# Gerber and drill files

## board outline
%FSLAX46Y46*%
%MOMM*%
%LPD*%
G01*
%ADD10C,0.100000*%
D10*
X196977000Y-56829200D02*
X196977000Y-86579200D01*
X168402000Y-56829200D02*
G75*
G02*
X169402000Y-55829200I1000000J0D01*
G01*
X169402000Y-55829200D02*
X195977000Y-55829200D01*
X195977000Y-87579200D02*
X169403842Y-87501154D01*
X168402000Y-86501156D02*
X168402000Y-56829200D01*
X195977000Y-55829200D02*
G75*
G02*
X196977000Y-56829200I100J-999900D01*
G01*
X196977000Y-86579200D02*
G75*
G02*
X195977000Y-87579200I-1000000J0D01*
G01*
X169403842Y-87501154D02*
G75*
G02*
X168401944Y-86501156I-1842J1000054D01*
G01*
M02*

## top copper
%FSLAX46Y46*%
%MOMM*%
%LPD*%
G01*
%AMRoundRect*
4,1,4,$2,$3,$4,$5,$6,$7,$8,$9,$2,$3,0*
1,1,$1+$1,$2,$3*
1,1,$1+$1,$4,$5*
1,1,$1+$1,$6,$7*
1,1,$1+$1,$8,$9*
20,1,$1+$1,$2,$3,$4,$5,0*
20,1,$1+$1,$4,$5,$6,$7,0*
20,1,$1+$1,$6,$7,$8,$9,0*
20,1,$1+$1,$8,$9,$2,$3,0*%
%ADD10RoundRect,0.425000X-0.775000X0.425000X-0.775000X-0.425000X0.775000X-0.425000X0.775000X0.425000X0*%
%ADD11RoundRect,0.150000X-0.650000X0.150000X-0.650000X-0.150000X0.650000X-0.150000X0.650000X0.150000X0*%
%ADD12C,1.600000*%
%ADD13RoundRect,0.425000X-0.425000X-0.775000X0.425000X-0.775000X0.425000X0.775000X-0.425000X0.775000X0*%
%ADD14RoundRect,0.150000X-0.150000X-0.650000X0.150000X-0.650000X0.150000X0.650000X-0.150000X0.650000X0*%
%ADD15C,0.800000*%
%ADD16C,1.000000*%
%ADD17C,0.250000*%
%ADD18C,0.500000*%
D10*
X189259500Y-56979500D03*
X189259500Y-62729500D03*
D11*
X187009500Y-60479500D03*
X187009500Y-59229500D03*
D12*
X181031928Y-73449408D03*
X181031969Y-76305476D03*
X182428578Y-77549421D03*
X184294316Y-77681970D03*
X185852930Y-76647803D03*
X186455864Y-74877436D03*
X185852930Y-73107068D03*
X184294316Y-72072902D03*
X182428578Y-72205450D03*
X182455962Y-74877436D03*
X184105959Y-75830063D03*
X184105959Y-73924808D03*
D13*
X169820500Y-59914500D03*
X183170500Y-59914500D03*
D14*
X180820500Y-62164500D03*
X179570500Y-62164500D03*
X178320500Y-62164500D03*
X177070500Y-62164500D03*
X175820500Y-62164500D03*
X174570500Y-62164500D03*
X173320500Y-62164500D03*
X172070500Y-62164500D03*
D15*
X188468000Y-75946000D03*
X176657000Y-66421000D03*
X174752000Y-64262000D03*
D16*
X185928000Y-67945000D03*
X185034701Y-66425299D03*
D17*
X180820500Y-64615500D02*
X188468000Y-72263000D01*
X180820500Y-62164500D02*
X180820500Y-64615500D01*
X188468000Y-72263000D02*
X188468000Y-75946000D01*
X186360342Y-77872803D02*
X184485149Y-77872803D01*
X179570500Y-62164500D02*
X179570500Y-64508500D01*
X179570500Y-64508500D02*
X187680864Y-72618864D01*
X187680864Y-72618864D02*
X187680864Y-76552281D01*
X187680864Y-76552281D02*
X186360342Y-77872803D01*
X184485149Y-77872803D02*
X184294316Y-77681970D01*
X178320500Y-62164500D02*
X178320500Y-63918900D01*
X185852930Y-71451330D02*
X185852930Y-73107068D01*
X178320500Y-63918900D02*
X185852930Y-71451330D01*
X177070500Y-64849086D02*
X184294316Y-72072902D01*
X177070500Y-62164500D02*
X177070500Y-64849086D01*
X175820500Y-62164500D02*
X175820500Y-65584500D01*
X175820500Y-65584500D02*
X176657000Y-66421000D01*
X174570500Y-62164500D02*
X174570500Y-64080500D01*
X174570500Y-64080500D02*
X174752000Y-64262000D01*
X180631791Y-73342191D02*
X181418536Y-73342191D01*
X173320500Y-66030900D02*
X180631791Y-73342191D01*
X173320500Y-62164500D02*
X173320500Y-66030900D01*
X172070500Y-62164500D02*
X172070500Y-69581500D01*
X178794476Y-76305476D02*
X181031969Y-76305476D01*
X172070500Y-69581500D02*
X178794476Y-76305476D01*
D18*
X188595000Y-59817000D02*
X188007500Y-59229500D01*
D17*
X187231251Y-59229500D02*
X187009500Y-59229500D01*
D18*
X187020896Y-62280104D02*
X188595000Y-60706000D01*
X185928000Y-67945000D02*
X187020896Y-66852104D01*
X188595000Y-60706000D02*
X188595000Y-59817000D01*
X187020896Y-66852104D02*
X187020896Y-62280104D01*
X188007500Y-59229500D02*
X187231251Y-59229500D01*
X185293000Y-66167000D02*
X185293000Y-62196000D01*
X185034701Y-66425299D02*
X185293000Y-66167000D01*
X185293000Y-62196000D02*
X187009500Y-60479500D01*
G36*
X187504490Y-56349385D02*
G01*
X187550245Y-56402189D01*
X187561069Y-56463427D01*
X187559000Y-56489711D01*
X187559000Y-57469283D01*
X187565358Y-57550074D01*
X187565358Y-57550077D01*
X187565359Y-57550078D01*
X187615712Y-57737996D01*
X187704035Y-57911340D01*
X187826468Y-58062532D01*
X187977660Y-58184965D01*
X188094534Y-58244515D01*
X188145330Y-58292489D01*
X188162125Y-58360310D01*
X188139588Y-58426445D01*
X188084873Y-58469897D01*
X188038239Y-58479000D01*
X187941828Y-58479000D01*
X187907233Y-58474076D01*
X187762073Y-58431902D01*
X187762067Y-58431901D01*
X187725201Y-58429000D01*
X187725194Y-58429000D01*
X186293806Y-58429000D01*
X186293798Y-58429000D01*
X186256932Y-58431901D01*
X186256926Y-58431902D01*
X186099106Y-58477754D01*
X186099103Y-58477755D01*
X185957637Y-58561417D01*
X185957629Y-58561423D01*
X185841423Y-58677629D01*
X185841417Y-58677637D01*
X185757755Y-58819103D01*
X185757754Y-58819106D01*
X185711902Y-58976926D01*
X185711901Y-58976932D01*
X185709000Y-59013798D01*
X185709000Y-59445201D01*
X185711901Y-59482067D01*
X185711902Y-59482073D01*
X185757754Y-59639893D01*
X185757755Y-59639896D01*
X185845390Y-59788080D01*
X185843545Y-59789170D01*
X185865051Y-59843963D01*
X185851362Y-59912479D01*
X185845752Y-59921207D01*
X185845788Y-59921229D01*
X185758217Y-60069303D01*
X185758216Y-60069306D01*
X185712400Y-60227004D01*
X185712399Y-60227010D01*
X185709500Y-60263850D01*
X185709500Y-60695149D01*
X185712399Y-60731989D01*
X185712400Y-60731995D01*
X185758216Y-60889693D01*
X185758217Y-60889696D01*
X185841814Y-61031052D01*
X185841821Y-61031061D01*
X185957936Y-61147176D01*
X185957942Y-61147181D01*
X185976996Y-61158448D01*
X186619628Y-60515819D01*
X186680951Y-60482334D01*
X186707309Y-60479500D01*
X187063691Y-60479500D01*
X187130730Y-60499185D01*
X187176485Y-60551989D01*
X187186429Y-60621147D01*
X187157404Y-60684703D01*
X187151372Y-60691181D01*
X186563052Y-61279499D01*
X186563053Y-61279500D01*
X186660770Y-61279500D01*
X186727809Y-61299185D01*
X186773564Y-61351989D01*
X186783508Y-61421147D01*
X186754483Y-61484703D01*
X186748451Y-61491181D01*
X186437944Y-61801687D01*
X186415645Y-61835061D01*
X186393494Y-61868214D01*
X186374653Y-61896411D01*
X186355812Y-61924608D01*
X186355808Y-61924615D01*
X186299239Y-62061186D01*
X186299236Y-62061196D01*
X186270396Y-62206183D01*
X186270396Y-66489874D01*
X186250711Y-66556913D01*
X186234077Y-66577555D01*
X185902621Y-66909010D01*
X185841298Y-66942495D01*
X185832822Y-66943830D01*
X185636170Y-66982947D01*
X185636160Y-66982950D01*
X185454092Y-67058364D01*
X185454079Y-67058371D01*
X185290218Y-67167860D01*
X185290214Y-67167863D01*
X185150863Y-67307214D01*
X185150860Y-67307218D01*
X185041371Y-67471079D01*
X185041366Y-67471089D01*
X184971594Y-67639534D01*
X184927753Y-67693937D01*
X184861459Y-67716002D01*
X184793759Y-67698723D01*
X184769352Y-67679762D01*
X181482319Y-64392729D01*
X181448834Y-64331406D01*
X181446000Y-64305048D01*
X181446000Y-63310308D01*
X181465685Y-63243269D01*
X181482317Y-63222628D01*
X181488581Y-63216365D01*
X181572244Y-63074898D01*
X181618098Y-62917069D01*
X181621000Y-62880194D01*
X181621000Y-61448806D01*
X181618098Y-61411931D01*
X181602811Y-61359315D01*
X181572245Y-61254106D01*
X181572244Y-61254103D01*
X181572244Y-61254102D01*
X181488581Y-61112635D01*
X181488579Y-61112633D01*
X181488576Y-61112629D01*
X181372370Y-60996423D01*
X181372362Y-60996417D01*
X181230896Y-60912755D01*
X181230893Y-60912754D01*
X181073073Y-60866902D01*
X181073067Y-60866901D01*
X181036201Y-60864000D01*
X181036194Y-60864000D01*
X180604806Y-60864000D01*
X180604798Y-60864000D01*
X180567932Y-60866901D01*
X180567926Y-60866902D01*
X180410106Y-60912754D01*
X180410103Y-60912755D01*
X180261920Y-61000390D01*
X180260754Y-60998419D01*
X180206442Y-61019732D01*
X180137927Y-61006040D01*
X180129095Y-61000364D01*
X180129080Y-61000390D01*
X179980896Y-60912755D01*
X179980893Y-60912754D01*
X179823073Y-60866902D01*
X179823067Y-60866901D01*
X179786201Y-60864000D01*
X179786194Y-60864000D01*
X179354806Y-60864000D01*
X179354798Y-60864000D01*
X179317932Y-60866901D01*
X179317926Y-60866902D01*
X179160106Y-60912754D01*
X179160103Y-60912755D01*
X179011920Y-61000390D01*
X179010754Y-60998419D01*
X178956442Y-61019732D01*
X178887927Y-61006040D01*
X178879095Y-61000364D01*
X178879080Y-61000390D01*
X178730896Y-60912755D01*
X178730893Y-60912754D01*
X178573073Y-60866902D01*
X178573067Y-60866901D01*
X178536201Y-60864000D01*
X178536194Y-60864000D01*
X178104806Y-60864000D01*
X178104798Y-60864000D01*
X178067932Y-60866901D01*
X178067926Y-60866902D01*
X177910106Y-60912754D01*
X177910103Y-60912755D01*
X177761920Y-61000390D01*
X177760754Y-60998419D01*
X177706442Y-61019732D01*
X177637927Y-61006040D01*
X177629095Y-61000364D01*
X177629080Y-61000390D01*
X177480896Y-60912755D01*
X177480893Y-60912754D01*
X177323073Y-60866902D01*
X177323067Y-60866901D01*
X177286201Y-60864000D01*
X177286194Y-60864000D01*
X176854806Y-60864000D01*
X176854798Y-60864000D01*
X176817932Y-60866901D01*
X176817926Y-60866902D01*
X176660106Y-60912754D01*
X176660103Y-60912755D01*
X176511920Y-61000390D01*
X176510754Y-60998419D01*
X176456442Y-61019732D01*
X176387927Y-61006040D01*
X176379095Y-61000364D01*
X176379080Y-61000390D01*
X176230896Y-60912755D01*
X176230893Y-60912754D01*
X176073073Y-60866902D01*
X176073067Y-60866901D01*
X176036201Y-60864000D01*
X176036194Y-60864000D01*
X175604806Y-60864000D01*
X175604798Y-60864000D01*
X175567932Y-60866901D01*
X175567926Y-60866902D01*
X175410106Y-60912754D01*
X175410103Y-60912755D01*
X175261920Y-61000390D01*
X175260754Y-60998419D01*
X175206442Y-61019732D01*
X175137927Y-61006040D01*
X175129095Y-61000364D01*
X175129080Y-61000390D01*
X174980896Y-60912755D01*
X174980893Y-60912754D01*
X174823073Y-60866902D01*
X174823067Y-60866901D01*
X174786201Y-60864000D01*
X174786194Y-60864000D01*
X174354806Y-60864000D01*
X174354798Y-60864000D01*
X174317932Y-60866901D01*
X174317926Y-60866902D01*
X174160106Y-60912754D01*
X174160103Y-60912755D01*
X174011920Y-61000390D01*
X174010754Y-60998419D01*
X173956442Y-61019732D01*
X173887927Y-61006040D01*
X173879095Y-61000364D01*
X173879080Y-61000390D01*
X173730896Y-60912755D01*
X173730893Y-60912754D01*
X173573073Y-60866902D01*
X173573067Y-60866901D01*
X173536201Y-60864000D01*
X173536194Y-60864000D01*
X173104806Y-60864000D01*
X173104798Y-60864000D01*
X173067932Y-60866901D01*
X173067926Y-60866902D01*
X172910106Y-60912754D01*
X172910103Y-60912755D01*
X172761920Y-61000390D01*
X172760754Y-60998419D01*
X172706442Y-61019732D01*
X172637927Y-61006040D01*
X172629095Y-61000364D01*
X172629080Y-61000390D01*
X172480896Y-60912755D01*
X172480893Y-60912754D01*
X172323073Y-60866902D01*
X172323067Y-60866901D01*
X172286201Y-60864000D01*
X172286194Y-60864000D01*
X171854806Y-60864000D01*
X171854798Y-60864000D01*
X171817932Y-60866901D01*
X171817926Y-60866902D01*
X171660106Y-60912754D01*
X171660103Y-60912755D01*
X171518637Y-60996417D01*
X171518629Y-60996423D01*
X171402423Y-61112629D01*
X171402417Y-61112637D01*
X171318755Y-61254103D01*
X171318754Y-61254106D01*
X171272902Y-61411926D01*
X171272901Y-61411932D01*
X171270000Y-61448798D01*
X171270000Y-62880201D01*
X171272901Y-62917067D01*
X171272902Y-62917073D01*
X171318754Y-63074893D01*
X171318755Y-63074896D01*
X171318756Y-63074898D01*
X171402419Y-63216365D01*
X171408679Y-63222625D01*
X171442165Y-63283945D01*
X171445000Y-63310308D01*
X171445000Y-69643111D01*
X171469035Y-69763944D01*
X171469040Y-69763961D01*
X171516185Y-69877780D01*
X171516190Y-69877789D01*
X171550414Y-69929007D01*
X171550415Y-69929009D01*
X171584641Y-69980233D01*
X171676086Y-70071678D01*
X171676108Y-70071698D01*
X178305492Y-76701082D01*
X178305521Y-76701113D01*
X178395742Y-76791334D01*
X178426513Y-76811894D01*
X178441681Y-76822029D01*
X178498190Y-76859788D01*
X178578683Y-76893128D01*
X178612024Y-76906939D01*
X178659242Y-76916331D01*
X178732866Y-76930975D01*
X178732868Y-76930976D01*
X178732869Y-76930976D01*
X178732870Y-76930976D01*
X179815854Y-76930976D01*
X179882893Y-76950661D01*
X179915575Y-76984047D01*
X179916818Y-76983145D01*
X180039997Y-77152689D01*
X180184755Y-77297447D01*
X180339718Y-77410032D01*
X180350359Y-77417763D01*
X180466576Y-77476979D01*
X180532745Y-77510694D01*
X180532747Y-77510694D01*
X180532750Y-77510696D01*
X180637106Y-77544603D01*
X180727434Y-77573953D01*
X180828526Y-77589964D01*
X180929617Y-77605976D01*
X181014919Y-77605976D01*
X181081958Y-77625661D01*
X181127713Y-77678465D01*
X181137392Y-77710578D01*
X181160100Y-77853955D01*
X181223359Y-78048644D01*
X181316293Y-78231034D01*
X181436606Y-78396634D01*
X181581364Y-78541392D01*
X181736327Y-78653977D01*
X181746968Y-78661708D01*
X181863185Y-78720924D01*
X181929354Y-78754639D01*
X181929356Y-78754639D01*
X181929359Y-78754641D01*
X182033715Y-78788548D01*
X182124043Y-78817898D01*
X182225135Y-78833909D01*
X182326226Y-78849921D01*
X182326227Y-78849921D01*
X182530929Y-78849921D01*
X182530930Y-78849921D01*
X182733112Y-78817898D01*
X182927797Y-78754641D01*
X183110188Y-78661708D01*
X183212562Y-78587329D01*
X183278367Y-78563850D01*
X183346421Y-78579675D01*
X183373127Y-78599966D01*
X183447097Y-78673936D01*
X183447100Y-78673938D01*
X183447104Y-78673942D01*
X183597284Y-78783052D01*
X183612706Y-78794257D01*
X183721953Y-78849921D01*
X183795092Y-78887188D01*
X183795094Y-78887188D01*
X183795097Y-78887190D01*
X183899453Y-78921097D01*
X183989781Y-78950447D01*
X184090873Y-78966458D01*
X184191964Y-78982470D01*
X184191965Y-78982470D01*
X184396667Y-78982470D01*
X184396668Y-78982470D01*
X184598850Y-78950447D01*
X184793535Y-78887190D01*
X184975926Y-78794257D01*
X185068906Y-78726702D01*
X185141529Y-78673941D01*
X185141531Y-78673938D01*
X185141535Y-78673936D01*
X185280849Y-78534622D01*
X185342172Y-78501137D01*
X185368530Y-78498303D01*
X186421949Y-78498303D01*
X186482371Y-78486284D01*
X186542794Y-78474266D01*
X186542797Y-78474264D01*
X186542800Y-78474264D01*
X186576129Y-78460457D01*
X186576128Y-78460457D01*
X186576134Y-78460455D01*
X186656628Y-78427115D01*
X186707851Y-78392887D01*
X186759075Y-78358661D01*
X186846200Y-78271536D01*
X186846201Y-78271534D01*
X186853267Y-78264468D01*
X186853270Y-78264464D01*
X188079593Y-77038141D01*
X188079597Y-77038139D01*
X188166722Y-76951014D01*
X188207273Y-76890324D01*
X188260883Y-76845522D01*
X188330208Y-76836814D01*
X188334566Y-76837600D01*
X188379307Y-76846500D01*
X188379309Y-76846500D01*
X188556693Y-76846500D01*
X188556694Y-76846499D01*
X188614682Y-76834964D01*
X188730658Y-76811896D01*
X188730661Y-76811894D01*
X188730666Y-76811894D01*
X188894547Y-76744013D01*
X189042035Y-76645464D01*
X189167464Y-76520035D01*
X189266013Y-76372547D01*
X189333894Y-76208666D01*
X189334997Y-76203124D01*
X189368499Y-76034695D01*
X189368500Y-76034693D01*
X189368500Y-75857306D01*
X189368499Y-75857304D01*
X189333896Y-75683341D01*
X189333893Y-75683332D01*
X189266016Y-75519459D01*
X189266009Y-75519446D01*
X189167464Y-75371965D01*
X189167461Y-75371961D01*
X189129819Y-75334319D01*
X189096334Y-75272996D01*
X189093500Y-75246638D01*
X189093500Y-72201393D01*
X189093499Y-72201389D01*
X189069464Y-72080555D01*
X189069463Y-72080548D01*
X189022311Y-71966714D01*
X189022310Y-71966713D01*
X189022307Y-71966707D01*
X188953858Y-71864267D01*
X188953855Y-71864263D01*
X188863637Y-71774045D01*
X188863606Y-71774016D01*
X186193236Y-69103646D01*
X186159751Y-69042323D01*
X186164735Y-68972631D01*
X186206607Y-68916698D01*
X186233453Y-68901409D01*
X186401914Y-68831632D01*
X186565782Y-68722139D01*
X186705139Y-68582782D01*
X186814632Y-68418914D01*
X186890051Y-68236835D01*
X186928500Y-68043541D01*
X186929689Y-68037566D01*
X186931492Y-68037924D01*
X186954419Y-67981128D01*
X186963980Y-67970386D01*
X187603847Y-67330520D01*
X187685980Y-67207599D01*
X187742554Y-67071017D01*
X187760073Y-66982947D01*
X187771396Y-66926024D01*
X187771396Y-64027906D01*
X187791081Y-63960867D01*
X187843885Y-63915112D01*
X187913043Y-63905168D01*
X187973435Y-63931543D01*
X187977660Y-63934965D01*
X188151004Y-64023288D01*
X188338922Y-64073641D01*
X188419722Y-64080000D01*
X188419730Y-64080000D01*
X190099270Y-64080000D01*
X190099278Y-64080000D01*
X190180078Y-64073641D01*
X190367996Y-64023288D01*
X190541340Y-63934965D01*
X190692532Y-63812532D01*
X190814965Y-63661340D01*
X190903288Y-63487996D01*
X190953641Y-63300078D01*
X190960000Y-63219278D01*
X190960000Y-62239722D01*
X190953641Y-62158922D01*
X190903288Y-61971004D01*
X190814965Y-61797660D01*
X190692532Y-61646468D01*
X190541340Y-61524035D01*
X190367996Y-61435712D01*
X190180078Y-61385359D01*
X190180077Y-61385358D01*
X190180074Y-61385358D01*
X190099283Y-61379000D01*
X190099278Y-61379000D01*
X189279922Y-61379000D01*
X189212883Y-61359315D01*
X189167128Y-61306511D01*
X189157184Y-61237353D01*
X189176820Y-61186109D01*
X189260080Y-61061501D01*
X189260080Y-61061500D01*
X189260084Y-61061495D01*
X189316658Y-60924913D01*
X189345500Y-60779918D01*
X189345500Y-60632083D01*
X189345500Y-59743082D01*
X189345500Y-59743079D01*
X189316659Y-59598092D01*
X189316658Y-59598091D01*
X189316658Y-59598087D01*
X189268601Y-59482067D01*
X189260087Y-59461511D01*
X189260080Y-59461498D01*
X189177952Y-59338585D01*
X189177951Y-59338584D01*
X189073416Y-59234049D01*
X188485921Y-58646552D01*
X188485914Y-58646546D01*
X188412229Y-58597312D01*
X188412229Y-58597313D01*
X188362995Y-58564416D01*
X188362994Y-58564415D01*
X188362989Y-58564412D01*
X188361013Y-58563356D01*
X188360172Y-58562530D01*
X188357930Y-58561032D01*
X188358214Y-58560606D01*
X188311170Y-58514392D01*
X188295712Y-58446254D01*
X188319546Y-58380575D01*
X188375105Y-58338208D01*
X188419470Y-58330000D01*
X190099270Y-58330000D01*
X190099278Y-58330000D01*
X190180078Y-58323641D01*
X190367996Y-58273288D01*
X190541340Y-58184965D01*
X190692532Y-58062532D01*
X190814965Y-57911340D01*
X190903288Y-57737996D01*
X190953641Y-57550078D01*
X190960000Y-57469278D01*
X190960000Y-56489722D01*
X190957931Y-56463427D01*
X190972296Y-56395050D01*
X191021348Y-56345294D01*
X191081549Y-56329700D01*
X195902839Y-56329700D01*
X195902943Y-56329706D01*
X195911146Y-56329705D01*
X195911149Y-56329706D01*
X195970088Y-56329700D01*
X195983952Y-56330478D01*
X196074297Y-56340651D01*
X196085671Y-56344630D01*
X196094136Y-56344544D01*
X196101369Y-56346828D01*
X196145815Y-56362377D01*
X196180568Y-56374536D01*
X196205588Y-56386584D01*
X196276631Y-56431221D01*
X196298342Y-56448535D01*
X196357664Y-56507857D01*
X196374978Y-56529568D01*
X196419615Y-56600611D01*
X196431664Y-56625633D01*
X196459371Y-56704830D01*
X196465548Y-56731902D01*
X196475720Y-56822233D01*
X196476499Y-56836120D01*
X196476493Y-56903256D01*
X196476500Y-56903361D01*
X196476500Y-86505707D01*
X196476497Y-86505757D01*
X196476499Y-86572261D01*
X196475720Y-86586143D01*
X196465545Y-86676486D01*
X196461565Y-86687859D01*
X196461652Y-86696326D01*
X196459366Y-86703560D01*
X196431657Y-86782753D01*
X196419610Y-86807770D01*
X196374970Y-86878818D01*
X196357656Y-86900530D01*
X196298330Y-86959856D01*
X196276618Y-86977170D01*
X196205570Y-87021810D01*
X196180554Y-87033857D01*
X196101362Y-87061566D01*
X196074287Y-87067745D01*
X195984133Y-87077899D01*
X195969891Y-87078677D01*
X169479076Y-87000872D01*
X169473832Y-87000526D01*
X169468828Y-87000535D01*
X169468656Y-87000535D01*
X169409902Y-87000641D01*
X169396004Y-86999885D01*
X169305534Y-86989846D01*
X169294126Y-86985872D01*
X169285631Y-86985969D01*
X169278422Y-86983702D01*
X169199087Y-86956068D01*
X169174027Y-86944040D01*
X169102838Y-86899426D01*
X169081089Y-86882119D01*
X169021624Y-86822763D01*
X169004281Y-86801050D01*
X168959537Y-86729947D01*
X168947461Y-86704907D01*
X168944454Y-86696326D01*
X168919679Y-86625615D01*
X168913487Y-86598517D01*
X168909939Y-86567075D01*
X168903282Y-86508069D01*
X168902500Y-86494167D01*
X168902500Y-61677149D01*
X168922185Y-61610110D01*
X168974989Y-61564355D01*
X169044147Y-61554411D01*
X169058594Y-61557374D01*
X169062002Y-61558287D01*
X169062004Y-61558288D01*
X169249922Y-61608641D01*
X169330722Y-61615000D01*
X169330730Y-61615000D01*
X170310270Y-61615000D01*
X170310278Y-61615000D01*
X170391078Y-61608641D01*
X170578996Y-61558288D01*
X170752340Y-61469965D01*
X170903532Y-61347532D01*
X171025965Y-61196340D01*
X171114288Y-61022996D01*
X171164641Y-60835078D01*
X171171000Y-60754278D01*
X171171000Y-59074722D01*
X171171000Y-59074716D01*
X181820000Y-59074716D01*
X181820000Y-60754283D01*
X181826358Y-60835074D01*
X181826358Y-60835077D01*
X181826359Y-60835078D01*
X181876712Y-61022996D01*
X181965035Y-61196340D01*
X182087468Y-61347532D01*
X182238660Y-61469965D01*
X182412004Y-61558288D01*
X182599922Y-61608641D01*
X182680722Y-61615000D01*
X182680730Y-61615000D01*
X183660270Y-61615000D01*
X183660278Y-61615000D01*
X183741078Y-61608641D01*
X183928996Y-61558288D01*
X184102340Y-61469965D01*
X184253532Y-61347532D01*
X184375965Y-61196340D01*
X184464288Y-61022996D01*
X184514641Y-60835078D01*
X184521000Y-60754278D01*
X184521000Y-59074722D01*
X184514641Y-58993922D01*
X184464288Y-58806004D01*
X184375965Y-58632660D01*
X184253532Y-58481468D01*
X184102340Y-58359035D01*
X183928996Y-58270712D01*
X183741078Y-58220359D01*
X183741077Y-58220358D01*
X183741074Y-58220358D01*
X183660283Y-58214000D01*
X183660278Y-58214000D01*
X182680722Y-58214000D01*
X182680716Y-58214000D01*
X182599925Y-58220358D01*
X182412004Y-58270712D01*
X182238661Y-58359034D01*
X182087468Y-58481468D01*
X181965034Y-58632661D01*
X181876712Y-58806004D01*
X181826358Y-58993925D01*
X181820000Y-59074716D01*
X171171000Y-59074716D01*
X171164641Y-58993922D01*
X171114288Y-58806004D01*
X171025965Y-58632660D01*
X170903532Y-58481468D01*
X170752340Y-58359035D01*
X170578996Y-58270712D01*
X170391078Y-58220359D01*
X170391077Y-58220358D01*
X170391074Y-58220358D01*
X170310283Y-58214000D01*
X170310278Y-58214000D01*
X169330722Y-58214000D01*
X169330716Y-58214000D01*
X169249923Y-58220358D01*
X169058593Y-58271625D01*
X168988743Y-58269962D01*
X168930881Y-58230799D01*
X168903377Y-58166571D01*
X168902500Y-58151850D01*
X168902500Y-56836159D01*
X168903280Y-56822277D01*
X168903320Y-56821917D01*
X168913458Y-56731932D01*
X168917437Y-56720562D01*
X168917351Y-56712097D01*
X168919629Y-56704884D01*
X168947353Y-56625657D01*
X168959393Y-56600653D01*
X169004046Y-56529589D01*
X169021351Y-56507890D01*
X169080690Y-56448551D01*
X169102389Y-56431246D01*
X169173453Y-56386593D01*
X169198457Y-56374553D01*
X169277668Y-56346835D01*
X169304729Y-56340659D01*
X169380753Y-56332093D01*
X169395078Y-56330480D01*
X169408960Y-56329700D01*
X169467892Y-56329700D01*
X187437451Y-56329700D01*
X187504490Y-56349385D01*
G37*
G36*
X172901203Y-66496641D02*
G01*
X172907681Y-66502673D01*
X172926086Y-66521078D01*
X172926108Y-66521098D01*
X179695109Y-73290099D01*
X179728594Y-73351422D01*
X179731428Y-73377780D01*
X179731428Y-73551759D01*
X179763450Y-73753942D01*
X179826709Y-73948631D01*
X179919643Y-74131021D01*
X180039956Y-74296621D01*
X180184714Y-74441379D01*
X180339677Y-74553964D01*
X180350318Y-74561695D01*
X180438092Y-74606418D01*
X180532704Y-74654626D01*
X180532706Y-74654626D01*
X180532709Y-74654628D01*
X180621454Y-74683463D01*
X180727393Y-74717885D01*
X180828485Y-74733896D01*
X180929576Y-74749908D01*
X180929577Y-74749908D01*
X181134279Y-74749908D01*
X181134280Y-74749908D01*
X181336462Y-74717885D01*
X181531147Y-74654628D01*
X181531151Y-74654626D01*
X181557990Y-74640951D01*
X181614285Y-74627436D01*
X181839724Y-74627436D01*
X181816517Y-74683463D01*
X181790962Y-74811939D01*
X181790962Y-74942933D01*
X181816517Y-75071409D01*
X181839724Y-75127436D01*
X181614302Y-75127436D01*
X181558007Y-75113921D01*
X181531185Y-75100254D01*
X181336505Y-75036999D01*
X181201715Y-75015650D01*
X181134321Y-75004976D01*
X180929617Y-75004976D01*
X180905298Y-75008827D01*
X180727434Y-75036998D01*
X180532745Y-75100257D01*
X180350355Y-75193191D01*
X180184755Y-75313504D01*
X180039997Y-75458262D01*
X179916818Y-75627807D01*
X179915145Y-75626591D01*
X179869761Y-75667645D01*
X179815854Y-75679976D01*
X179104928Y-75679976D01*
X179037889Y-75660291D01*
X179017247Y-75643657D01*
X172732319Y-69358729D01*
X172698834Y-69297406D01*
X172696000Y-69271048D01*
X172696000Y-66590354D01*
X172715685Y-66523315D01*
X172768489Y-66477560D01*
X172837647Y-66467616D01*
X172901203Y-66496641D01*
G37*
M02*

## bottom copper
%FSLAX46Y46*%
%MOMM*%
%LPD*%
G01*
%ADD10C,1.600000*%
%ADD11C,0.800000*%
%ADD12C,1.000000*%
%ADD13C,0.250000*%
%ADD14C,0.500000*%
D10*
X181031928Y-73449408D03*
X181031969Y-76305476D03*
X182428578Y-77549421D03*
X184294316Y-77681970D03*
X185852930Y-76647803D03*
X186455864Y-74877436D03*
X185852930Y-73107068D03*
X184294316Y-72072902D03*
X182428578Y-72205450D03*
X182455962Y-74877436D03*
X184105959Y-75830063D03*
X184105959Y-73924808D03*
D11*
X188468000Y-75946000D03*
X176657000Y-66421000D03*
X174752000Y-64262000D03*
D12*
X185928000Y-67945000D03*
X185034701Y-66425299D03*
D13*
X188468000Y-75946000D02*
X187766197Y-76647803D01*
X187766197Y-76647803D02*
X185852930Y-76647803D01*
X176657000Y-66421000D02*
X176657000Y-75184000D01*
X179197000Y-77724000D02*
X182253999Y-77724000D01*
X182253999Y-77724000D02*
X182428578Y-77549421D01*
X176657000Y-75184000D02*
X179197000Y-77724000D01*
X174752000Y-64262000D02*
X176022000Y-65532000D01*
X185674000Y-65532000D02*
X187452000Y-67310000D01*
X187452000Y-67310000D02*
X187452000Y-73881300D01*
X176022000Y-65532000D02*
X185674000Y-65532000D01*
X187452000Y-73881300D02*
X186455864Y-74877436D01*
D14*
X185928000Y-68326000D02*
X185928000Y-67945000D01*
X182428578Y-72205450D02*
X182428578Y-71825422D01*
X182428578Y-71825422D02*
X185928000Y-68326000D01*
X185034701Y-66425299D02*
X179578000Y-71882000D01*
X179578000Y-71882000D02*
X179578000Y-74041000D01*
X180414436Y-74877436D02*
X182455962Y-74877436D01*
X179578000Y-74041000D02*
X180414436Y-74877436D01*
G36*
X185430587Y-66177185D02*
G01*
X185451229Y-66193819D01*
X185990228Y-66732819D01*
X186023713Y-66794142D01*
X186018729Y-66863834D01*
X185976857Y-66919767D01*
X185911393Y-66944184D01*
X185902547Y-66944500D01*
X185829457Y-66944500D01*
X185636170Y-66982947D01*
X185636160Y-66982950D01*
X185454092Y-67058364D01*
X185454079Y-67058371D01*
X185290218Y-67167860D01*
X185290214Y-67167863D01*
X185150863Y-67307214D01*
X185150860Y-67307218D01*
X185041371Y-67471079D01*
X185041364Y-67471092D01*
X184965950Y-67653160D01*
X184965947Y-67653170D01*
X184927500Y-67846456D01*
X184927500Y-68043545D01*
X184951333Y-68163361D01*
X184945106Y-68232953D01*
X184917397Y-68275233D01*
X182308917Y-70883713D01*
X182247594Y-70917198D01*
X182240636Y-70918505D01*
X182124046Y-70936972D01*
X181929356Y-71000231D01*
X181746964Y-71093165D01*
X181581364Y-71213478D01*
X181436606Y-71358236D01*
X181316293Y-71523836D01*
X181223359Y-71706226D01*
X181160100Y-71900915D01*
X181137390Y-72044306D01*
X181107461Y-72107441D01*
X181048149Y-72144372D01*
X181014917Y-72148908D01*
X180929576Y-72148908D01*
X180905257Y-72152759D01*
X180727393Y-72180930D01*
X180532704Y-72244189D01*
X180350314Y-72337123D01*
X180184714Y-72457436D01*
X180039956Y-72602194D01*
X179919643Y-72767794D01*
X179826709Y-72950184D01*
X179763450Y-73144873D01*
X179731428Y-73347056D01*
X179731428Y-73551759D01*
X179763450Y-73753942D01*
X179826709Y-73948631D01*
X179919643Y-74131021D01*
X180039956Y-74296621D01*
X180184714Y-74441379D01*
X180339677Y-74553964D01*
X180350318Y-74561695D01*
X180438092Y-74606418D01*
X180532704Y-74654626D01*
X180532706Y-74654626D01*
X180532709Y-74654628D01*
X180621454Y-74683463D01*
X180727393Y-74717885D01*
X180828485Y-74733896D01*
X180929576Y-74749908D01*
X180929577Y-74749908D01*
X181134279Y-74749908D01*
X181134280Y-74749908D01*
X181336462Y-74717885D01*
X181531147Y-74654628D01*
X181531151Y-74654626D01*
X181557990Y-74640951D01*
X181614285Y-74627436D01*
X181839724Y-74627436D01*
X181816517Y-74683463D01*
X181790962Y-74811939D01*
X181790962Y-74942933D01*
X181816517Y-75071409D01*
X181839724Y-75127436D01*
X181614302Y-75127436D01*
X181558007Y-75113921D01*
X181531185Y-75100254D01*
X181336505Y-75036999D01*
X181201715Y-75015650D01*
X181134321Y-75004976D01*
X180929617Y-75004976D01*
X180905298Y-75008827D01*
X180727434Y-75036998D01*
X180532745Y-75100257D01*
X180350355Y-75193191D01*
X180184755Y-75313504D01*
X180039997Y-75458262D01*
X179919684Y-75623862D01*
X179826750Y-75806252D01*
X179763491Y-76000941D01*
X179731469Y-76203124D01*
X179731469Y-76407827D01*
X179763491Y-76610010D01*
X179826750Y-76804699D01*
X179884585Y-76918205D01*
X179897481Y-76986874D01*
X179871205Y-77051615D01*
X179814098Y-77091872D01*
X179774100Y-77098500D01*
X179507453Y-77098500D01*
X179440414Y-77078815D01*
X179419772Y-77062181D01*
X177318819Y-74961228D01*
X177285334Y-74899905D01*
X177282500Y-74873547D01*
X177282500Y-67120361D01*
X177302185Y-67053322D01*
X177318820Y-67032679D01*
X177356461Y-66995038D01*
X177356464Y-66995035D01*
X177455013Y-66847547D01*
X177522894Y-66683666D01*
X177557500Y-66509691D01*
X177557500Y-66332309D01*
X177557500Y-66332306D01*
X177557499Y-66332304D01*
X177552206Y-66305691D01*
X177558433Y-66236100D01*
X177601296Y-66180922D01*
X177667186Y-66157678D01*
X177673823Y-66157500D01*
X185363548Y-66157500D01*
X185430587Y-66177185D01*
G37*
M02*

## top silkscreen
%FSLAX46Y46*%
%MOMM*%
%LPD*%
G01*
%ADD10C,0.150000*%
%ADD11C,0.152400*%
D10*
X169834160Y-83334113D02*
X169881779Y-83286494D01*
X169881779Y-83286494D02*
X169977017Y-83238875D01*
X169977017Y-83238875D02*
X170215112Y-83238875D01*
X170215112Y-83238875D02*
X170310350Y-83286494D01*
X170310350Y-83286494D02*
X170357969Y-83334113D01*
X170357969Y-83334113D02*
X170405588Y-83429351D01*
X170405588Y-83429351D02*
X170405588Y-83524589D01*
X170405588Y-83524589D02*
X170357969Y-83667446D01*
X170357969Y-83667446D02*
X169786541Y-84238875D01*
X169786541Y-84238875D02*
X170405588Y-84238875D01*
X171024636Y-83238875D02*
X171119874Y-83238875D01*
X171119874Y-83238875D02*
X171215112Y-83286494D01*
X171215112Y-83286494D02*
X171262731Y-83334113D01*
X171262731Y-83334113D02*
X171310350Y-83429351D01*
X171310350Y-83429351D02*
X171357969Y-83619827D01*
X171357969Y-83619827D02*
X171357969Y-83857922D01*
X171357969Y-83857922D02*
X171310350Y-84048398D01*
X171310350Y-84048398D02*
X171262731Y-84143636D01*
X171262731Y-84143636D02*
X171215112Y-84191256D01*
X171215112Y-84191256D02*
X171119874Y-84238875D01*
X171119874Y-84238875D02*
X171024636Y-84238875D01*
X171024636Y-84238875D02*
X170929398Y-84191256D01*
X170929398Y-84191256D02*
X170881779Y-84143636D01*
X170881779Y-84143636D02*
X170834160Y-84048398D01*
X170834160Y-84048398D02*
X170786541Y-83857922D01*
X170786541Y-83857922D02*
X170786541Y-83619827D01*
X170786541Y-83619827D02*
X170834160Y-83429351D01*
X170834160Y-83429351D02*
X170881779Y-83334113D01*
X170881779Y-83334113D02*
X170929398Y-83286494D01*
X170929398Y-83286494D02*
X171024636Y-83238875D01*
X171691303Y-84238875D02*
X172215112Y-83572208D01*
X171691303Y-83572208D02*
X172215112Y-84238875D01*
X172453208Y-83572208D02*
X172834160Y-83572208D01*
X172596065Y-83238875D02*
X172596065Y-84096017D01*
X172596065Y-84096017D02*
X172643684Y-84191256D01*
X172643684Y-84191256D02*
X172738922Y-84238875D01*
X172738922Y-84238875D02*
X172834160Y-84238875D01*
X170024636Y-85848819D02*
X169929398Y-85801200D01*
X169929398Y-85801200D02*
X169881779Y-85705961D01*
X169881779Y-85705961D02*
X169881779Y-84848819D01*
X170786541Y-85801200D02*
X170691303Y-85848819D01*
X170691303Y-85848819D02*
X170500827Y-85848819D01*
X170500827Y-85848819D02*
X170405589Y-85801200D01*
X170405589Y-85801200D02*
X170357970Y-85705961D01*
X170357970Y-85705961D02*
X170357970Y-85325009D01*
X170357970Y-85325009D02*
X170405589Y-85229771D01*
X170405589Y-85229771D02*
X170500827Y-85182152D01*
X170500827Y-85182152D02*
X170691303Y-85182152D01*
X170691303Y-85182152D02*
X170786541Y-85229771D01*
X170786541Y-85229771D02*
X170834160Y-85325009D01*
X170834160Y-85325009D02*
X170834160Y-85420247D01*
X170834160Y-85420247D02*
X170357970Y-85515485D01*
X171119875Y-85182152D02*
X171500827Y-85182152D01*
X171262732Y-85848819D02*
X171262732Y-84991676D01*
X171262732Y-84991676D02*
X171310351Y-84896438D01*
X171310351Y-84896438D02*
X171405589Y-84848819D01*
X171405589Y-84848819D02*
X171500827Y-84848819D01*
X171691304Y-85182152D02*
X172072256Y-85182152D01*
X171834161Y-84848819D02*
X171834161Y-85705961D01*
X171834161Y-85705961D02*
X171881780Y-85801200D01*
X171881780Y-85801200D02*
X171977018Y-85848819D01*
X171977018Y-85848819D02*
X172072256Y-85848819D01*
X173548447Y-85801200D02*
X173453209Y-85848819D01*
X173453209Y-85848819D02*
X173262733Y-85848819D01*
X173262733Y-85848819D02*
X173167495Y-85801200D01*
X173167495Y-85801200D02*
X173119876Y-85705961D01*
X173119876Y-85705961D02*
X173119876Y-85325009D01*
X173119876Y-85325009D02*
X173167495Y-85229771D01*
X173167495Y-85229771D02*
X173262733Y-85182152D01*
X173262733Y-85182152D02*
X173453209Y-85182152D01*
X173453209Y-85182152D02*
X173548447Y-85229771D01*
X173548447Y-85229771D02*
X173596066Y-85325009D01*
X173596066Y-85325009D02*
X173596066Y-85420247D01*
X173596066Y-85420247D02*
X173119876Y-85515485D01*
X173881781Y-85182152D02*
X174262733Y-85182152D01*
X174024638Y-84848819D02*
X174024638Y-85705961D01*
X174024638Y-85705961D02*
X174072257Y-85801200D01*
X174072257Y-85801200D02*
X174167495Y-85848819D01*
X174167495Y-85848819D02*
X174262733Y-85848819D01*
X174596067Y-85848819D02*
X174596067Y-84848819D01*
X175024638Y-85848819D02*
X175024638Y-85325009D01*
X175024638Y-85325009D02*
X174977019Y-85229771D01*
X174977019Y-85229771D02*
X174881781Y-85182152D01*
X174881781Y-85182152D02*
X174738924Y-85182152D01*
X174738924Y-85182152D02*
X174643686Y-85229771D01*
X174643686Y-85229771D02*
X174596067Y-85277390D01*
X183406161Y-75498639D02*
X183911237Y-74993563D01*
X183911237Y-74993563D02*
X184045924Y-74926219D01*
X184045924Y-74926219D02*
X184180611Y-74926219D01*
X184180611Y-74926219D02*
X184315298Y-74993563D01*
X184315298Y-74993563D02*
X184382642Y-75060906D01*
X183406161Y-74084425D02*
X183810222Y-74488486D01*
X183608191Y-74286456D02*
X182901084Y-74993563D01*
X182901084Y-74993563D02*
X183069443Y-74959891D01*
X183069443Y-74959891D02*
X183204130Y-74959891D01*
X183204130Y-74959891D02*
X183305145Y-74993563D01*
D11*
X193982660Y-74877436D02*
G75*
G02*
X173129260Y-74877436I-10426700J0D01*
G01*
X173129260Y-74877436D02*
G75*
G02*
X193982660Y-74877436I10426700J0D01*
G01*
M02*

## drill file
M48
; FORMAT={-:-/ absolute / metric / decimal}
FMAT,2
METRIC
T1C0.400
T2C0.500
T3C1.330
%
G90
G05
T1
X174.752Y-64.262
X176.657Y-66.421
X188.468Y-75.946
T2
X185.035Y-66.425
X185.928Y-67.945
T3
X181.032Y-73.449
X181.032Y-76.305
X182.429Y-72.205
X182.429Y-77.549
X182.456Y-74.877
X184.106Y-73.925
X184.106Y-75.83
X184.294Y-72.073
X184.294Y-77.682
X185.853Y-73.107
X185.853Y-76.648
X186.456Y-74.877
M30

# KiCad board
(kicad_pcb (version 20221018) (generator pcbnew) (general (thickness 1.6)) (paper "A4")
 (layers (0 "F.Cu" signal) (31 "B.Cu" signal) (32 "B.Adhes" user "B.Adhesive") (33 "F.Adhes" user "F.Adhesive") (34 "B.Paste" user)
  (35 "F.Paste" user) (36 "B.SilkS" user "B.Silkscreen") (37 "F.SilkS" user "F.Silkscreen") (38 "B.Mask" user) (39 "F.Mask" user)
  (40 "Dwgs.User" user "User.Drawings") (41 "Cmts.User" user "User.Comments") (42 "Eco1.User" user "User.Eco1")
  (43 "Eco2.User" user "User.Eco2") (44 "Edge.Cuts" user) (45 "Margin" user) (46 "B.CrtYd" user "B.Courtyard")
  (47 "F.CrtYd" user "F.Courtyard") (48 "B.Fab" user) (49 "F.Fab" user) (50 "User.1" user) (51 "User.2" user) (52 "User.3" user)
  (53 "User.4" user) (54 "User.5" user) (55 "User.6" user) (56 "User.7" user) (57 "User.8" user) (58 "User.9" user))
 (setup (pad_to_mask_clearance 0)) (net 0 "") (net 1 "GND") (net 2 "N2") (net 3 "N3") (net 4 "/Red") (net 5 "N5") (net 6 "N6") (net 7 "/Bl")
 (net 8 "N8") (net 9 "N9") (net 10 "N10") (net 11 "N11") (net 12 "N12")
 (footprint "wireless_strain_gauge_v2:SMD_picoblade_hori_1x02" (layer "F.Cu") (at 186.2095 56.1295 -90)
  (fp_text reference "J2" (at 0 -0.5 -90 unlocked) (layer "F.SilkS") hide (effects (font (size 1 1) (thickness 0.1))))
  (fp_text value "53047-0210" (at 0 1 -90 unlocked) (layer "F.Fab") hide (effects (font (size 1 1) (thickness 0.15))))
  (pad "" smd roundrect (at 0.85 -3.05 270) (size 1.7 2.4) (layers "F.Cu" "F.Paste" "F.Mask") (roundrect_rratio 0.25)
   (thermal_bridge_angle 45))
  (pad "" smd roundrect (at 6.6 -3.05 270) (size 1.7 2.4) (layers "F.Cu" "F.Paste" "F.Mask") (roundrect_rratio 0.25)
   (thermal_bridge_angle 45))
  (pad "1" smd roundrect (at 4.35 -0.8 270) (size 0.6 1.6) (layers "F.Cu" "F.Paste" "F.Mask") (roundrect_rratio 0.25) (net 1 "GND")
   (thermal_bridge_angle 45))
  (pad "2" smd roundrect (at 3.1 -0.8 270) (size 0.6 1.6) (layers "F.Cu" "F.Paste" "F.Mask") (roundrect_rratio 0.25) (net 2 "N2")
   (thermal_bridge_angle 45)))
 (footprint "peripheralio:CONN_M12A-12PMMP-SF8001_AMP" (layer "F.Cu") (at 181.031928 73.449408 135)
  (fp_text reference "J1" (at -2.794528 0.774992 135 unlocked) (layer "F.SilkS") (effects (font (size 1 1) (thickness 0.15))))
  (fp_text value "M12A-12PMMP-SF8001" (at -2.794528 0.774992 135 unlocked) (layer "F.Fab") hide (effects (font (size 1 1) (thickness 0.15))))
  (fp_circle (center -2.794528 0.774992) (end 7.632172 0.774992) (stroke (width 0.1524) (type solid)) (fill none) (layer "F.SilkS"))
  (pad "1" thru_hole circle (at 0 0 135) (size 1.6 1.6) (drill 1.33) (layers "*.Cu" "*.Mask") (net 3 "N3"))
  (pad "2" thru_hole circle (at -2.019574 -2.019516 135) (size 1.6 1.6) (drill 1.33) (layers "*.Cu" "*.Mask") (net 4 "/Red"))
  (pad "3" thru_hole circle (at -3.886728 -1.911566 225) (size 1.6 1.6) (drill 1.33) (layers "*.Cu" "*.Mask") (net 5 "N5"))
  (pad "4" thru_hole circle (at -5.29973 -0.686016 135) (size 1.6 1.6) (drill 1.33) (layers "*.Cu" "*.Mask") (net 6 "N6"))
  (pad "5" thru_hole circle (at -5.67057 1.147356 135) (size 1.6 1.6) (drill 1.33) (layers "*.Cu" "*.Mask") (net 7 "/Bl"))
  (pad "6" thru_hole circle (at -4.84507 2.825534 135) (size 1.6 1.6) (drill 1.33) (layers "*.Cu" "*.Mask") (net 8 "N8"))
  (pad "7" thru_hole circle (at -3.166892 3.651034 135) (size 1.6 1.6) (drill 1.33) (layers "*.Cu" "*.Mask") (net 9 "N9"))
  (pad "8" thru_hole circle (at -1.33352 3.280194 135) (size 1.6 1.6) (drill 1.33) (layers "*.Cu" "*.Mask") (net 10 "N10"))
  (pad "9" thru_hole circle (at -0.10797 1.867192 135) (size 1.6 1.6) (drill 1.33) (layers "*.Cu" "*.Mask") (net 2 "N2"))
  (pad "10" thru_hole circle (at -2.016712 -0.002824 135) (size 1.6 1.6) (drill 1.33) (layers "*.Cu" "*.Mask") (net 1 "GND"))
  (pad "11" thru_hole circle (at -3.857046 0.490291 345) (size 1.6 1.6) (drill 1.33) (layers "*.Cu" "*.Mask") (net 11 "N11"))
  (pad "12" thru_hole circle (at -2.509827 1.83751 15) (size 1.6 1.6) (drill 1.33) (layers "*.Cu" "*.Mask") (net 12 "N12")))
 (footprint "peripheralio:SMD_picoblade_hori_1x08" (layer "F.Cu") (at 168.9705 62.9645)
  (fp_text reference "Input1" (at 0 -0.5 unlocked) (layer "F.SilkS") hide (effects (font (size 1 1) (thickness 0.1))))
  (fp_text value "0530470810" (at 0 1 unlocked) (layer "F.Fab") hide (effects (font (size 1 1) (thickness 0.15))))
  (pad "" smd roundrect (at 0.85 -3.05) (size 1.7 2.4) (layers "F.Cu" "F.Paste" "F.Mask") (roundrect_rratio 0.25) (thermal_bridge_angle 45))
  (pad "" smd roundrect (at 14.2 -3.05) (size 1.7 2.4) (layers "F.Cu" "F.Paste" "F.Mask") (roundrect_rratio 0.25) (thermal_bridge_angle 45))
  (pad "1" smd roundrect (at 11.85 -0.8) (size 0.6 1.6) (layers "F.Cu" "F.Paste" "F.Mask") (roundrect_rratio 0.25) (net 7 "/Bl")
   (thermal_bridge_angle 45))
  (pad "2" smd roundrect (at 10.6 -0.8) (size 0.6 1.6) (layers "F.Cu" "F.Paste" "F.Mask") (roundrect_rratio 0.25) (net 6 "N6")
   (thermal_bridge_angle 45))
  (pad "3" smd roundrect (at 9.35 -0.8) (size 0.6 1.6) (layers "F.Cu" "F.Paste" "F.Mask") (roundrect_rratio 0.25) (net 9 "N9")
   (thermal_bridge_angle 45))
  (pad "4" smd roundrect (at 8.1 -0.8) (size 0.6 1.6) (layers "F.Cu" "F.Paste" "F.Mask") (roundrect_rratio 0.25) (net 10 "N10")
   (thermal_bridge_angle 45))
  (pad "5" smd roundrect (at 6.85 -0.8) (size 0.6 1.6) (layers "F.Cu" "F.Paste" "F.Mask") (roundrect_rratio 0.25) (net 5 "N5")
   (thermal_bridge_angle 45))
  (pad "6" smd roundrect (at 5.6 -0.8) (size 0.6 1.6) (layers "F.Cu" "F.Paste" "F.Mask") (roundrect_rratio 0.25) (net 8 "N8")
   (thermal_bridge_angle 45))
  (pad "7" smd roundrect (at 4.35 -0.8) (size 0.6 1.6) (layers "F.Cu" "F.Paste" "F.Mask") (roundrect_rratio 0.25) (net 3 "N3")
   (thermal_bridge_angle 45))
  (pad "8" smd roundrect (at 3.1 -0.8) (size 0.6 1.6) (layers "F.Cu" "F.Paste" "F.Mask") (roundrect_rratio 0.25) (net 4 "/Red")
   (thermal_bridge_angle 45)))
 (gr_line (start 196.977 56.8292) (end 196.977 86.5792) (stroke (width 0.1) (type default)) (layer "Edge.Cuts"))
 (gr_arc (start 168.402 56.8292) (mid 168.694893 56.122093) (end 169.402 55.8292) (stroke (width 0.1) (type default)) (layer "Edge.Cuts"))
 (gr_line (start 169.402 55.8292) (end 195.977 55.8292) (stroke (width 0.1) (type default)) (layer "Edge.Cuts"))
 (gr_line (start 195.977 87.5792) (end 169.403842 87.501154) (stroke (width 0.1) (type default)) (layer "Edge.Cuts"))
 (gr_line (start 168.402 86.501156) (end 168.402 56.8292) (stroke (width 0.1) (type default)) (layer "Edge.Cuts"))
 (gr_arc (start 195.977 55.8292) (mid 196.684131 56.122069) (end 196.977 56.8292) (stroke (width 0.1) (type default)) (layer "Edge.Cuts"))
 (gr_arc (start 196.977 86.5792) (mid 196.684121 87.286321) (end 195.977 87.5792) (stroke (width 0.1) (type default)) (layer "Edge.Cuts"))
 (gr_arc (start 169.403842 87.501154) (mid 168.695561 87.208911) (end 168.402 86.501156) (stroke (width 0.1) (type default))
  (layer "Edge.Cuts"))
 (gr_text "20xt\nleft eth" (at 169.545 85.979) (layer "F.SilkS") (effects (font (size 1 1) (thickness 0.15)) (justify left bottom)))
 (segment (start 180.8205 64.6155) (end 188.468 72.263) (width 0.25) (layer "F.Cu") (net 7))
 (segment (start 180.8205 62.1645) (end 180.8205 64.6155) (width 0.25) (layer "F.Cu") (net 7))
 (segment (start 188.468 72.263) (end 188.468 75.946) (width 0.25) (layer "F.Cu") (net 7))
 (via (at 188.468 75.946) (size 0.8) (drill 0.4) (layers "F.Cu" "B.Cu") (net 7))
 (segment (start 188.468 75.946) (end 187.766197 76.647803) (width 0.25) (layer "B.Cu") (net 7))
 (segment (start 187.766197 76.647803) (end 185.85293 76.647803) (width 0.25) (layer "B.Cu") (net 7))
 (segment (start 186.360342 77.872803) (end 184.485149 77.872803) (width 0.25) (layer "F.Cu") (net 6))
 (segment (start 179.5705 62.1645) (end 179.5705 64.5085) (width 0.25) (layer "F.Cu") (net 6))
 (segment (start 179.5705 64.5085) (end 187.680864 72.618864) (width 0.25) (layer "F.Cu") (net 6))
 (segment (start 187.680864 72.618864) (end 187.680864 76.552281) (width 0.25) (layer "F.Cu") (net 6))
 (segment (start 187.680864 76.552281) (end 186.360342 77.872803) (width 0.25) (layer "F.Cu") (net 6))
 (segment (start 184.485149 77.872803) (end 184.294316 77.68197) (width 0.25) (layer "F.Cu") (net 6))
 (segment (start 178.3205 62.1645) (end 178.3205 63.9189) (width 0.25) (layer "F.Cu") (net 9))
 (segment (start 185.85293 71.45133) (end 185.85293 73.107068) (width 0.25) (layer "F.Cu") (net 9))
 (segment (start 178.3205 63.9189) (end 185.85293 71.45133) (width 0.25) (layer "F.Cu") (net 9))
 (segment (start 177.0705 64.849086) (end 184.294316 72.072902) (width 0.25) (layer "F.Cu") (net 10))
 (segment (start 177.0705 62.1645) (end 177.0705 64.849086) (width 0.25) (layer "F.Cu") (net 10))
 (segment (start 175.8205 62.1645) (end 175.8205 65.5845) (width 0.25) (layer "F.Cu") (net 5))
 (segment (start 175.8205 65.5845) (end 176.657 66.421) (width 0.25) (layer "F.Cu") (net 5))
 (via (at 176.657 66.421) (size 0.8) (drill 0.4) (layers "F.Cu" "B.Cu") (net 5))
 (segment (start 176.657 66.421) (end 176.657 75.184) (width 0.25) (layer "B.Cu") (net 5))
 (segment (start 179.197 77.724) (end 182.253999 77.724) (width 0.25) (layer "B.Cu") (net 5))
 (segment (start 182.253999 77.724) (end 182.428578 77.549421) (width 0.25) (layer "B.Cu") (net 5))
 (segment (start 176.657 75.184) (end 179.197 77.724) (width 0.25) (layer "B.Cu") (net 5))
 (segment (start 174.5705 62.1645) (end 174.5705 64.0805) (width 0.25) (layer "F.Cu") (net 8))
 (segment (start 174.5705 64.0805) (end 174.752 64.262) (width 0.25) (layer "F.Cu") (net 8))
 (via (at 174.752 64.262) (size 0.8) (drill 0.4) (layers "F.Cu" "B.Cu") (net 8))
 (segment (start 174.752 64.262) (end 176.022 65.532) (width 0.25) (layer "B.Cu") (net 8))
 (segment (start 185.674 65.532) (end 187.452 67.31) (width 0.25) (layer "B.Cu") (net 8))
 (segment (start 187.452 67.31) (end 187.452 73.8813) (width 0.25) (layer "B.Cu") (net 8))
 (segment (start 176.022 65.532) (end 185.674 65.532) (width 0.25) (layer "B.Cu") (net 8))
 (segment (start 187.452 73.8813) (end 186.455864 74.877436) (width 0.25) (layer "B.Cu") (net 8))
 (segment (start 180.631791 73.342191) (end 181.418536 73.342191) (width 0.25) (layer "F.Cu") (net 3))
 (segment (start 173.3205 66.0309) (end 180.631791 73.342191) (width 0.25) (layer "F.Cu") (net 3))
 (segment (start 173.3205 62.1645) (end 173.3205 66.0309) (width 0.25) (layer "F.Cu") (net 3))
 (segment (start 172.0705 62.1645) (end 172.0705 69.5815) (width 0.25) (layer "F.Cu") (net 4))
 (segment (start 178.794476 76.305476) (end 181.031969 76.305476) (width 0.25) (layer "F.Cu") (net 4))
 (segment (start 172.0705 69.5815) (end 178.794476 76.305476) (width 0.25) (layer "F.Cu") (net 4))
 (segment (start 188.595 59.817) (end 188.0075 59.2295) (width 0.5) (layer "F.Cu") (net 2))
 (segment (start 187.231251 59.2295) (end 187.0095 59.2295) (width 0.25) (layer "F.Cu") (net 2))
 (segment (start 187.020896 62.280104) (end 188.595 60.706) (width 0.5) (layer "F.Cu") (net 2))
 (segment (start 185.928 67.945) (end 187.020896 66.852104) (width 0.5) (layer "F.Cu") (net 2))
 (segment (start 188.595 60.706) (end 188.595 59.817) (width 0.5) (layer "F.Cu") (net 2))
 (segment (start 187.020896 66.852104) (end 187.020896 62.280104) (width 0.5) (layer "F.Cu") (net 2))
 (segment (start 188.0075 59.2295) (end 187.231251 59.2295) (width 0.5) (layer "F.Cu") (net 2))
 (via (at 185.928 67.945) (size 1) (drill 0.5) (layers "F.Cu" "B.Cu") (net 2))
 (segment (start 185.928 68.326) (end 185.928 67.945) (width 0.5) (layer "B.Cu") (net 2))
 (segment (start 182.428578 72.20545) (end 182.428578 71.825422) (width 0.5) (layer "B.Cu") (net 2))
 (segment (start 182.428578 71.825422) (end 185.928 68.326) (width 0.5) (layer "B.Cu") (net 2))
 (segment (start 185.293 66.167) (end 185.293 62.196) (width 0.5) (layer "F.Cu") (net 1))
 (segment (start 185.034701 66.425299) (end 185.293 66.167) (width 0.5) (layer "F.Cu") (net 1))
 (segment (start 185.293 62.196) (end 187.0095 60.4795) (width 0.5) (layer "F.Cu") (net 1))
 (via (at 185.034701 66.425299) (size 1) (drill 0.5) (layers "F.Cu" "B.Cu") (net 1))
 (segment (start 185.034701 66.425299) (end 179.578 71.882) (width 0.5) (layer "B.Cu") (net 1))
 (segment (start 179.578 71.882) (end 179.578 74.041) (width 0.5) (layer "B.Cu") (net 1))
 (segment (start 180.414436 74.877436) (end 182.455962 74.877436) (width 0.5) (layer "B.Cu") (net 1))
 (segment (start 179.578 74.041) (end 180.414436 74.877436) (width 0.5) (layer "B.Cu") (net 1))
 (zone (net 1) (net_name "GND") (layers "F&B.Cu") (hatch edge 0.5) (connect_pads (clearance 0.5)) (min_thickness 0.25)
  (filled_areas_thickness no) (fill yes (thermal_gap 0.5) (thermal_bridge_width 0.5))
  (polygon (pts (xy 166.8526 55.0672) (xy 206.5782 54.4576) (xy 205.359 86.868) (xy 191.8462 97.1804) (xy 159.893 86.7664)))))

